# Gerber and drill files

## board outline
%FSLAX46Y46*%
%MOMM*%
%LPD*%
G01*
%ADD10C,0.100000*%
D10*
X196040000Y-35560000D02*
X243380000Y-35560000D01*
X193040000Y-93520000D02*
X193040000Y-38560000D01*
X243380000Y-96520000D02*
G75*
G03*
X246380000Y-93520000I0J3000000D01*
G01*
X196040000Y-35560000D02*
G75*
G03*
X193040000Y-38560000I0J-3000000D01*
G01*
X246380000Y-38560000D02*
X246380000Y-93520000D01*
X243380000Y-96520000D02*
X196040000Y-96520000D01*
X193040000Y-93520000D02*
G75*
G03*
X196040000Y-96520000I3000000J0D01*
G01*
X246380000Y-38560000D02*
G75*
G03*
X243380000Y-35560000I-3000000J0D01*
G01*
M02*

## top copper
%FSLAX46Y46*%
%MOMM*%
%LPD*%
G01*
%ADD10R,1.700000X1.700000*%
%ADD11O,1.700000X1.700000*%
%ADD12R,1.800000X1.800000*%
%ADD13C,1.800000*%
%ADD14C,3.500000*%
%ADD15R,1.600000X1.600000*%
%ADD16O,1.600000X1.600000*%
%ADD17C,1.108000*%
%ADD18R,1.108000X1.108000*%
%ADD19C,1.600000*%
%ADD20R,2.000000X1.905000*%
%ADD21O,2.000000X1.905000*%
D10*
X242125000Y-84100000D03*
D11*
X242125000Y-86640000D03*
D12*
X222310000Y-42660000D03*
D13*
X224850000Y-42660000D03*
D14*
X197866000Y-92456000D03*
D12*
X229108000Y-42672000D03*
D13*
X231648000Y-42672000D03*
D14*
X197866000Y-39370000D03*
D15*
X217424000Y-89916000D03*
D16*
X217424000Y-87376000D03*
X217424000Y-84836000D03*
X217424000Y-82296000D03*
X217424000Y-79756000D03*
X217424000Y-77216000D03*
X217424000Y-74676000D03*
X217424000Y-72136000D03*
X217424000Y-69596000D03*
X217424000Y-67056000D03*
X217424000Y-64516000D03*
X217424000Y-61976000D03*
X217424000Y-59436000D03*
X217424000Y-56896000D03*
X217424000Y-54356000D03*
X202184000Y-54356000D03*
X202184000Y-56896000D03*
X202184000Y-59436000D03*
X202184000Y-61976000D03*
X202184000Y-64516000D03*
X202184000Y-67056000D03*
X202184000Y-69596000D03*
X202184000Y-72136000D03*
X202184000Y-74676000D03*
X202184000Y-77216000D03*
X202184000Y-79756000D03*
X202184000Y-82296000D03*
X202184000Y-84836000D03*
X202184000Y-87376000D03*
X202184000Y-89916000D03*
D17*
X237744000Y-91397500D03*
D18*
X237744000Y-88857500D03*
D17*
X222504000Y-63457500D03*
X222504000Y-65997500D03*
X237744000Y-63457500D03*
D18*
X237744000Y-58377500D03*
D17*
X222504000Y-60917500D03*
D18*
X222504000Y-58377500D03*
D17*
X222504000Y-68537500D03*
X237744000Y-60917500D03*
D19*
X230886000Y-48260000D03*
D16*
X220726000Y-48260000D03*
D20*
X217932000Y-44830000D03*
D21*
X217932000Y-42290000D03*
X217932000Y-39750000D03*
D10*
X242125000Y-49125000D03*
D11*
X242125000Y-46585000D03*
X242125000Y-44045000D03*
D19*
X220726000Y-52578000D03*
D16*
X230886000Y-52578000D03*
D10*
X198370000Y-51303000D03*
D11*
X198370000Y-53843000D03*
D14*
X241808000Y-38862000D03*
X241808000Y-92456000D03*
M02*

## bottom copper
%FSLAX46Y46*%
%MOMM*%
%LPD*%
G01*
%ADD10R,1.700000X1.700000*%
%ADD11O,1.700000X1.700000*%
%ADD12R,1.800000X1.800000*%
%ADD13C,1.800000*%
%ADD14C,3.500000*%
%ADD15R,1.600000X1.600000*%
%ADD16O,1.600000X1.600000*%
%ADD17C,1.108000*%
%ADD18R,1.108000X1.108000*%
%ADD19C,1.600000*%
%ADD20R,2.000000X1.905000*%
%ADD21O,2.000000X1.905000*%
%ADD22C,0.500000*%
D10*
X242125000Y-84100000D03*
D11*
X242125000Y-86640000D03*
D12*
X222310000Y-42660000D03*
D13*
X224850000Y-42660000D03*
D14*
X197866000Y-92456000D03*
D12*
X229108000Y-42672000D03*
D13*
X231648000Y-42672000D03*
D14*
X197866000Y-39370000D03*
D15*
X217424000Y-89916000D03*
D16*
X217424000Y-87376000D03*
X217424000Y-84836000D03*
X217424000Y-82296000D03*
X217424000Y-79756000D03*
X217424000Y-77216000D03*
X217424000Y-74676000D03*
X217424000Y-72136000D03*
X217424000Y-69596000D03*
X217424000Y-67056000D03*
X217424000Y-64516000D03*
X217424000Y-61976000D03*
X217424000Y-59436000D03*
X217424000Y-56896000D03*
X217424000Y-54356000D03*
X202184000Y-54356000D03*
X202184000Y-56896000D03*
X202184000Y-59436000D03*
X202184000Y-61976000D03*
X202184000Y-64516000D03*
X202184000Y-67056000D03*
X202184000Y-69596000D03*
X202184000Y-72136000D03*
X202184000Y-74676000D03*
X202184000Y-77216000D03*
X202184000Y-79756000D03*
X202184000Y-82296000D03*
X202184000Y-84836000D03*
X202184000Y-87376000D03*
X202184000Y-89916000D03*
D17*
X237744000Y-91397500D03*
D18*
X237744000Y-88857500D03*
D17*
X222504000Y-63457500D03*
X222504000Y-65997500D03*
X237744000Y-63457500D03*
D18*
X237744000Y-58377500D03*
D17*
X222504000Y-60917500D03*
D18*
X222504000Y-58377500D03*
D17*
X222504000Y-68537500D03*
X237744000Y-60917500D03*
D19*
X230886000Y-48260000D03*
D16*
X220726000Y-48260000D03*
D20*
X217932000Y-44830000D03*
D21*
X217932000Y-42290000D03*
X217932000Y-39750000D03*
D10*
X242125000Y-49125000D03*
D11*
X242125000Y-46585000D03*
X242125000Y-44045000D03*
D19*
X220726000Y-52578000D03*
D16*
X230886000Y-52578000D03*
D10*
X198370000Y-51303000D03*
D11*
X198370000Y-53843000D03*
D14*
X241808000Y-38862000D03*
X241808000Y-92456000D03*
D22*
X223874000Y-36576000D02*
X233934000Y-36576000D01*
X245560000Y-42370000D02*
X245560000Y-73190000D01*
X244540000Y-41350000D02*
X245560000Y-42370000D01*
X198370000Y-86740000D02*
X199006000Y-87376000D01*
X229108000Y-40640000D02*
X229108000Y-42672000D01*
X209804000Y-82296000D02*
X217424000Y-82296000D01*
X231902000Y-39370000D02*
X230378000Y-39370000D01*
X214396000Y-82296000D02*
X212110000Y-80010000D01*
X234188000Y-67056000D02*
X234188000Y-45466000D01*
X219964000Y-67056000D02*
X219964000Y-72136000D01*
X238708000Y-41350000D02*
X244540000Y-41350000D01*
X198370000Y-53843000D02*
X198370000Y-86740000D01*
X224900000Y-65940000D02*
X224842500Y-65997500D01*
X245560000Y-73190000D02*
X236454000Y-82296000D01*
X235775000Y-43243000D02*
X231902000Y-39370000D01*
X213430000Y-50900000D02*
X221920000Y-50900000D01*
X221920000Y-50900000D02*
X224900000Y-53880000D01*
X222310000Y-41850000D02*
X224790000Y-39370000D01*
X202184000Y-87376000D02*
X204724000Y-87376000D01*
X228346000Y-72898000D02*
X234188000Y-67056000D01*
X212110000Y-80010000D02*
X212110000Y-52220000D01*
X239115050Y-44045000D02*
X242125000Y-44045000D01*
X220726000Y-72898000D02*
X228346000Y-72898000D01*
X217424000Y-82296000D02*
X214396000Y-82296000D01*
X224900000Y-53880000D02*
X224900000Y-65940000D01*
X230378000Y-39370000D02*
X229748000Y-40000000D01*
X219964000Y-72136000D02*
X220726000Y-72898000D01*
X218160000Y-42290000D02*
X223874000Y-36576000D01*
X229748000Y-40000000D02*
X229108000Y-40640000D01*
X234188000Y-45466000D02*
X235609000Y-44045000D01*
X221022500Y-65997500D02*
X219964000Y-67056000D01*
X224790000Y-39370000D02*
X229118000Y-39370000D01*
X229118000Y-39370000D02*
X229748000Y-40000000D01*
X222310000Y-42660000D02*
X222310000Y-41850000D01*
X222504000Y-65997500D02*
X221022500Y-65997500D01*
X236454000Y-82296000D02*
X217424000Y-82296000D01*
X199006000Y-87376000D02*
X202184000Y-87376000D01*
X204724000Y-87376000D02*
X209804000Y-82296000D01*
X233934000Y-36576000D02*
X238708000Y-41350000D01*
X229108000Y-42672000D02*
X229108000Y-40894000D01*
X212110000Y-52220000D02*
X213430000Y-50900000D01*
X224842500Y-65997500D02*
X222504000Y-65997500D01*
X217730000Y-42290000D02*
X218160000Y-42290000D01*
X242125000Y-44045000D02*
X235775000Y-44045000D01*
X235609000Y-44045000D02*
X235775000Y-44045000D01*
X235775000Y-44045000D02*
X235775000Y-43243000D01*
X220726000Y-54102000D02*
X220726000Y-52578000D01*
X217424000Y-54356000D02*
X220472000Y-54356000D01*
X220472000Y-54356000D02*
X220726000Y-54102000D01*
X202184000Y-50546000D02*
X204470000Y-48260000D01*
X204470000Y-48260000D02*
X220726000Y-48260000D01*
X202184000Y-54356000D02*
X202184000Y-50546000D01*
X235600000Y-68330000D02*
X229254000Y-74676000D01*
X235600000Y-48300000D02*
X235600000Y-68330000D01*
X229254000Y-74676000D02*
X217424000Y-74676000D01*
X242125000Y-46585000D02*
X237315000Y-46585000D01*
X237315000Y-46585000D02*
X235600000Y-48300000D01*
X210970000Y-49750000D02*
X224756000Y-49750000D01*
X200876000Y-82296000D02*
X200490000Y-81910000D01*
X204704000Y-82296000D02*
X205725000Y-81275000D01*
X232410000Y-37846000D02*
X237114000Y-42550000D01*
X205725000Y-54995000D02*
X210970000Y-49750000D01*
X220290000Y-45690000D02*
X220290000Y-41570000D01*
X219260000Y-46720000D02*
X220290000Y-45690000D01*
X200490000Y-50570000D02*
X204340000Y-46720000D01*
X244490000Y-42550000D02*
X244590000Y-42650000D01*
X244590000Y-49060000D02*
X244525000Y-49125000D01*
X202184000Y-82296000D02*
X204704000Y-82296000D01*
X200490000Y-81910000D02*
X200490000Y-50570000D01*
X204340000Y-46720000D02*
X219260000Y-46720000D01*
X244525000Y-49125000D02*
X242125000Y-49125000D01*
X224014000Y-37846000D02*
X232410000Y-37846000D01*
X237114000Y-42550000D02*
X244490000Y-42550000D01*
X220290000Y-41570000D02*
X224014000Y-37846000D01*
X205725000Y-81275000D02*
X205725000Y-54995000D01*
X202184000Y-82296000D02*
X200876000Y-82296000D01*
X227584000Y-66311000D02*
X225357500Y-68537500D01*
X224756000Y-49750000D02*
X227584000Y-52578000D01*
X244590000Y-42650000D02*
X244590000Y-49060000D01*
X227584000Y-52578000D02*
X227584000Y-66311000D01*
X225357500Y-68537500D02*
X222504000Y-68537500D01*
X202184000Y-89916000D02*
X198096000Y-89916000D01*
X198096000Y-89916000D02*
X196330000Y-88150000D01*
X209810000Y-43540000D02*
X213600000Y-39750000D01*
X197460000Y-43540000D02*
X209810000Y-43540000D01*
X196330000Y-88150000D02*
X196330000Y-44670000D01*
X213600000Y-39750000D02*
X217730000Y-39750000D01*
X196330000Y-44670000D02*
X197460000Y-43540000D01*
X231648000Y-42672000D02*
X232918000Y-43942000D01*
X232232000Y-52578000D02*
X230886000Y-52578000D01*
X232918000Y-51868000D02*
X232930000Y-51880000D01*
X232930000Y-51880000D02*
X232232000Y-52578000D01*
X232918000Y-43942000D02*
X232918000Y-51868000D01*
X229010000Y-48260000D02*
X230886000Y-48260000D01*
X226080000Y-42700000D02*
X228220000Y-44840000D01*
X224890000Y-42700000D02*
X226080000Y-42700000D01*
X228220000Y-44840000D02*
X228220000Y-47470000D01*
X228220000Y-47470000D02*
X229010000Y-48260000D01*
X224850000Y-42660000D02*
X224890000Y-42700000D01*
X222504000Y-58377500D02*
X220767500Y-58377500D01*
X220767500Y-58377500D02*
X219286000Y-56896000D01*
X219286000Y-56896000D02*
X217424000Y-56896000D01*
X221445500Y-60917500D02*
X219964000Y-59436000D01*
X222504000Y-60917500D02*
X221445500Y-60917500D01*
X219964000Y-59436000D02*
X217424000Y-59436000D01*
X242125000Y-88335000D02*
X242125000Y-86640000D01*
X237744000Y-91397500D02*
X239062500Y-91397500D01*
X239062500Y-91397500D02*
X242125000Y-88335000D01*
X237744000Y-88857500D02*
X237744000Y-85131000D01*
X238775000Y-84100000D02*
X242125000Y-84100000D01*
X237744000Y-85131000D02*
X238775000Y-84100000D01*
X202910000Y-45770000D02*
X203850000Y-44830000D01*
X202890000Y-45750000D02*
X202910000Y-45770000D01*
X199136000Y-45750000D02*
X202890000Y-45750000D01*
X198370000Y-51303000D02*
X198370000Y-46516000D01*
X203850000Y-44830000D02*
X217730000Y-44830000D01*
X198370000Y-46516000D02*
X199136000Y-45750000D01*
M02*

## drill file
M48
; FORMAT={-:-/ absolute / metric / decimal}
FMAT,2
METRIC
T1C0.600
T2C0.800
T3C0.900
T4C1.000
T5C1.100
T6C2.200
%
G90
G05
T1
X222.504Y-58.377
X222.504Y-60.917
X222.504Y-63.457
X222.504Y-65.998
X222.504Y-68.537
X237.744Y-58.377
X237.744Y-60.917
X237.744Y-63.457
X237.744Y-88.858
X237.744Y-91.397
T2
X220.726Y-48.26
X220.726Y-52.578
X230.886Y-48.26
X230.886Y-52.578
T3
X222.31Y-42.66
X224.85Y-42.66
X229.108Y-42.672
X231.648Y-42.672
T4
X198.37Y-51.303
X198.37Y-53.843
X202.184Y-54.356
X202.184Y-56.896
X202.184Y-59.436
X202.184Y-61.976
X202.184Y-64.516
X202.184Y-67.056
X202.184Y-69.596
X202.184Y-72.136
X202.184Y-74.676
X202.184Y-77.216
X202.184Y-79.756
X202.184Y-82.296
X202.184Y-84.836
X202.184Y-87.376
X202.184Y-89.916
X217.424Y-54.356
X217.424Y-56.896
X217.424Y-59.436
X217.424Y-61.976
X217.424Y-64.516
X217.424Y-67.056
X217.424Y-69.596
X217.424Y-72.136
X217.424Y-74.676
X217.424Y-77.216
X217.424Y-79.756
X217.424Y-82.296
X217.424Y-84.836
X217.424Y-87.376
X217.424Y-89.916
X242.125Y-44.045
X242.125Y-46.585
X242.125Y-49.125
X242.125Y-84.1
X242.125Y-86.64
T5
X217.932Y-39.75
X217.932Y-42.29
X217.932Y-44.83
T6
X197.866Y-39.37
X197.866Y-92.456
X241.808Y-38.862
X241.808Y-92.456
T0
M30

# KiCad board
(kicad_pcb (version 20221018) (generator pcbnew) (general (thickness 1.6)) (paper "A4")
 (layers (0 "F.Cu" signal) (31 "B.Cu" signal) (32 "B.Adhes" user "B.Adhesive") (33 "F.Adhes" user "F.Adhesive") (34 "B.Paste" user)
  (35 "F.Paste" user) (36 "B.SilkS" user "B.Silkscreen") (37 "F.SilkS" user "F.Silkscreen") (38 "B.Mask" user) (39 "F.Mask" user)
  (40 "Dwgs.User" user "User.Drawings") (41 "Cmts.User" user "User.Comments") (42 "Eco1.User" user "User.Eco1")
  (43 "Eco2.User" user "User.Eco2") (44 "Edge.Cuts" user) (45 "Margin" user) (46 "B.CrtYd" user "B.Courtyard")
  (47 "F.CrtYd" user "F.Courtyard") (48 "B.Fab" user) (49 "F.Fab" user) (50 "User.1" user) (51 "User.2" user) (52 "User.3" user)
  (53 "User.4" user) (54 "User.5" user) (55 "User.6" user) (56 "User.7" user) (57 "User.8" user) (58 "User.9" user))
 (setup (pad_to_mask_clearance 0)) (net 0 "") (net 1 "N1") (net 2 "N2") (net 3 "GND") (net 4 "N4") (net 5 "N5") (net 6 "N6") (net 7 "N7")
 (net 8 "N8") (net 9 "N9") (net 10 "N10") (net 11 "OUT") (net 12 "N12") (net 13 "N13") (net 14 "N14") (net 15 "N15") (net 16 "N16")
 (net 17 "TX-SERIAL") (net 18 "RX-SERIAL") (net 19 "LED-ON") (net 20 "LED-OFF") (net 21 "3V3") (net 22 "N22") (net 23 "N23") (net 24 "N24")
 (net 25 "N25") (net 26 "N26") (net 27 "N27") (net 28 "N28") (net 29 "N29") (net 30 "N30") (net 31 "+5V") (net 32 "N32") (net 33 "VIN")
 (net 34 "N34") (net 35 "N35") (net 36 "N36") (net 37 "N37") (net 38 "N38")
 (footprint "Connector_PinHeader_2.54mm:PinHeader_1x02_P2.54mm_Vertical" (layer "F.Cu") (at 242.125 84.1)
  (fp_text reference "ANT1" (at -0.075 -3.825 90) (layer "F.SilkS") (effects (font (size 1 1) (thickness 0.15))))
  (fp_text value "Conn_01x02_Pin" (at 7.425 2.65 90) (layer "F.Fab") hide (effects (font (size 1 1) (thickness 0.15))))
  (pad "1" thru_hole rect (at 0 0) (size 1.7 1.7) (drill 1) (layers "*.Cu" "*.Mask") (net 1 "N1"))
  (pad "2" thru_hole oval (at 0 2.54) (size 1.7 1.7) (drill 1) (layers "*.Cu" "*.Mask") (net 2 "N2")))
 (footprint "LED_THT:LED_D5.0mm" (layer "F.Cu") (at 222.31 42.66)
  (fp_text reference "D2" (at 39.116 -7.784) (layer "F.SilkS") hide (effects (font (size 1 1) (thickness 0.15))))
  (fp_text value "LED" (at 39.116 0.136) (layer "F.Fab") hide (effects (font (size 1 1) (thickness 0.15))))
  (pad "1" thru_hole rect (at 0 0) (size 1.8 1.8) (drill 0.9) (layers "*.Cu" "*.Mask") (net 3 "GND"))
  (pad "2" thru_hole circle (at 2.54 0) (size 1.8 1.8) (drill 0.9) (layers "*.Cu" "*.Mask") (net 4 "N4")))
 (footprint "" (layer "F.Cu") (at 197.866 92.456)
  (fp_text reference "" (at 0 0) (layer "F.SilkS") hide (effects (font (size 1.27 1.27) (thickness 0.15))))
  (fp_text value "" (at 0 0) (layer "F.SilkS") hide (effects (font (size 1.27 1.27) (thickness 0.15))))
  (pad "1" thru_hole circle (at 0 0) (size 3.5 3.5) (drill 2.2) (layers "*.Cu" "*.Mask")))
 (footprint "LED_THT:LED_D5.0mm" (layer "F.Cu") (at 229.108 42.672)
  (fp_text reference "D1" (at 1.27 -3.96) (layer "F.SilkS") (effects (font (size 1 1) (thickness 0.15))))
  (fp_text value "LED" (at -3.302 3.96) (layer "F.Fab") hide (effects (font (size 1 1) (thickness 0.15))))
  (pad "1" thru_hole rect (at 0 0) (size 1.8 1.8) (drill 0.9) (layers "*.Cu" "*.Mask") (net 3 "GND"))
  (pad "2" thru_hole circle (at 2.54 0) (size 1.8 1.8) (drill 0.9) (layers "*.Cu" "*.Mask") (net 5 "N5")))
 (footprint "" (layer "F.Cu") (at 197.866 39.37)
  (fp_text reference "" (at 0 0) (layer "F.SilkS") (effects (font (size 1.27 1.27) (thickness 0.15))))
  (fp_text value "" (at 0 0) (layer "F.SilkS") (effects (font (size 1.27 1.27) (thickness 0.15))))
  (pad "1" thru_hole circle (at 0 0) (size 3.5 3.5) (drill 2.2) (layers "*.Cu" "*.Mask")))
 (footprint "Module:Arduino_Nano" (layer "F.Cu") (at 217.424 89.916 180)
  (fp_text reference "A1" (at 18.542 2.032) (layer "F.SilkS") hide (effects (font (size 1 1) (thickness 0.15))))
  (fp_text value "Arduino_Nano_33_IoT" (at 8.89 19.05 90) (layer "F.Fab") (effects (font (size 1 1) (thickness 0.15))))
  (pad "1" thru_hole rect (at 0 0 180) (size 1.6 1.6) (drill 1) (layers "*.Cu" "*.Mask") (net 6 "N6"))
  (pad "2" thru_hole oval (at 0 2.54 180) (size 1.6 1.6) (drill 1) (layers "*.Cu" "*.Mask") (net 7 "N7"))
  (pad "3" thru_hole oval (at 0 5.08 180) (size 1.6 1.6) (drill 1) (layers "*.Cu" "*.Mask") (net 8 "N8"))
  (pad "4" thru_hole oval (at 0 7.62 180) (size 1.6 1.6) (drill 1) (layers "*.Cu" "*.Mask") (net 3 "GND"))
  (pad "5" thru_hole oval (at 0 10.16 180) (size 1.6 1.6) (drill 1) (layers "*.Cu" "*.Mask") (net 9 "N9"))
  (pad "6" thru_hole oval (at 0 12.7 180) (size 1.6 1.6) (drill 1) (layers "*.Cu" "*.Mask") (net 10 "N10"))
  (pad "7" thru_hole oval (at 0 15.24 180) (size 1.6 1.6) (drill 1) (layers "*.Cu" "*.Mask") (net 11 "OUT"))
  (pad "8" thru_hole oval (at 0 17.78 180) (size 1.6 1.6) (drill 1) (layers "*.Cu" "*.Mask") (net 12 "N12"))
  (pad "9" thru_hole oval (at 0 20.32 180) (size 1.6 1.6) (drill 1) (layers "*.Cu" "*.Mask") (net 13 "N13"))
  (pad "10" thru_hole oval (at 0 22.86 180) (size 1.6 1.6) (drill 1) (layers "*.Cu" "*.Mask") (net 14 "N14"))
  (pad "11" thru_hole oval (at 0 25.4 180) (size 1.6 1.6) (drill 1) (layers "*.Cu" "*.Mask") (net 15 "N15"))
  (pad "12" thru_hole oval (at 0 27.94 180) (size 1.6 1.6) (drill 1) (layers "*.Cu" "*.Mask") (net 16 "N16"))
  (pad "13" thru_hole oval (at 0 30.48 180) (size 1.6 1.6) (drill 1) (layers "*.Cu" "*.Mask") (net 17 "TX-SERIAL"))
  (pad "14" thru_hole oval (at 0 33.02 180) (size 1.6 1.6) (drill 1) (layers "*.Cu" "*.Mask") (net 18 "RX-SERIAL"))
  (pad "15" thru_hole oval (at 0 35.56 180) (size 1.6 1.6) (drill 1) (layers "*.Cu" "*.Mask") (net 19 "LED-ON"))
  (pad "16" thru_hole oval (at 15.24 35.56 180) (size 1.6 1.6) (drill 1) (layers "*.Cu" "*.Mask") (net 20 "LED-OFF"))
  (pad "17" thru_hole oval (at 15.24 33.02 180) (size 1.6 1.6) (drill 1) (layers "*.Cu" "*.Mask") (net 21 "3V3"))
  (pad "18" thru_hole oval (at 15.24 30.48 180) (size 1.6 1.6) (drill 1) (layers "*.Cu" "*.Mask") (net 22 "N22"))
  (pad "19" thru_hole oval (at 15.24 27.94 180) (size 1.6 1.6) (drill 1) (layers "*.Cu" "*.Mask") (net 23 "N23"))
  (pad "20" thru_hole oval (at 15.24 25.4 180) (size 1.6 1.6) (drill 1) (layers "*.Cu" "*.Mask") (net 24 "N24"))
  (pad "21" thru_hole oval (at 15.24 22.86 180) (size 1.6 1.6) (drill 1) (layers "*.Cu" "*.Mask") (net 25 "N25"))
  (pad "22" thru_hole oval (at 15.24 20.32 180) (size 1.6 1.6) (drill 1) (layers "*.Cu" "*.Mask") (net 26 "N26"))
  (pad "23" thru_hole oval (at 15.24 17.78 180) (size 1.6 1.6) (drill 1) (layers "*.Cu" "*.Mask") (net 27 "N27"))
  (pad "24" thru_hole oval (at 15.24 15.24 180) (size 1.6 1.6) (drill 1) (layers "*.Cu" "*.Mask") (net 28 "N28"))
  (pad "25" thru_hole oval (at 15.24 12.7 180) (size 1.6 1.6) (drill 1) (layers "*.Cu" "*.Mask") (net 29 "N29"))
  (pad "26" thru_hole oval (at 15.24 10.16 180) (size 1.6 1.6) (drill 1) (layers "*.Cu" "*.Mask") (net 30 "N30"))
  (pad "27" thru_hole oval (at 15.24 7.62 180) (size 1.6 1.6) (drill 1) (layers "*.Cu" "*.Mask") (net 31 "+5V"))
  (pad "28" thru_hole oval (at 15.24 5.08 180) (size 1.6 1.6) (drill 1) (layers "*.Cu" "*.Mask") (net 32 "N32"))
  (pad "29" thru_hole oval (at 15.24 2.54 180) (size 1.6 1.6) (drill 1) (layers "*.Cu" "*.Mask") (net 3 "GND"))
  (pad "30" thru_hole oval (at 15.24 0 180) (size 1.6 1.6) (drill 1) (layers "*.Cu" "*.Mask") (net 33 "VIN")))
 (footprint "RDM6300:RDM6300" (layer "F.Cu") (at 230.124 74.8875 90)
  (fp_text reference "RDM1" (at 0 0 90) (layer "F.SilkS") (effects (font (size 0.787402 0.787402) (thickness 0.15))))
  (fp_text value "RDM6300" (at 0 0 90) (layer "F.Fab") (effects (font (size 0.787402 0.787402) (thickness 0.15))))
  (pad "ANT1" thru_hole circle (at -16.51 7.62 90) (size 1.108 1.108) (drill 0.6) (layers "*.Cu" "*.Mask") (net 2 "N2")
   (solder_mask_margin 0.102))
  (pad "ANT2" thru_hole rect (at -13.97 7.62 90) (size 1.108 1.108) (drill 0.6) (layers "*.Cu" "*.Mask") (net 1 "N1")
   (solder_mask_margin 0.102))
  (pad "D0" thru_hole circle (at 11.43 -7.62 90) (size 1.108 1.108) (drill 0.6) (layers "*.Cu" "*.Mask") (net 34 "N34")
   (solder_mask_margin 0.102))
  (pad "GND" thru_hole circle (at 8.89 -7.62 90) (size 1.108 1.108) (drill 0.6) (layers "*.Cu" "*.Mask") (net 3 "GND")
   (solder_mask_margin 0.102))
  (pad "GND1" thru_hole circle (at 11.43 7.62 90) (size 1.108 1.108) (drill 0.6) (layers "*.Cu" "*.Mask") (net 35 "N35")
   (solder_mask_margin 0.102))
  (pad "LED" thru_hole rect (at 16.51 7.62 90) (size 1.108 1.108) (drill 0.6) (layers "*.Cu" "*.Mask") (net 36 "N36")
   (solder_mask_margin 0.102))
  (pad "RX" thru_hole circle (at 13.97 -7.62 90) (size 1.108 1.108) (drill 0.6) (layers "*.Cu" "*.Mask") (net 17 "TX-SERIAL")
   (solder_mask_margin 0.102))
  (pad "TX" thru_hole rect (at 16.51 -7.62 90) (size 1.108 1.108) (drill 0.6) (layers "*.Cu" "*.Mask") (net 18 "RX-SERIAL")
   (solder_mask_margin 0.102))
  (pad "VCC" thru_hole circle (at 6.35 -7.62 90) (size 1.108 1.108) (drill 0.6) (layers "*.Cu" "*.Mask") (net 31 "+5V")
   (solder_mask_margin 0.102))
  (pad "VCC1" thru_hole circle (at 13.97 7.62 90) (size 1.108 1.108) (drill 0.6) (layers "*.Cu" "*.Mask") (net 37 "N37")
   (solder_mask_margin 0.102)))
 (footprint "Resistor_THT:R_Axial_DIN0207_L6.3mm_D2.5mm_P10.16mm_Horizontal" (layer "F.Cu") (at 230.886 48.26 180)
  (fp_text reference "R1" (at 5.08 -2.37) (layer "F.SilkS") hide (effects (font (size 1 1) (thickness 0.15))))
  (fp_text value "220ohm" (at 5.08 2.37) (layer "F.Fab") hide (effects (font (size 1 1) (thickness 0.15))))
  (pad "1" thru_hole circle (at 0 0 180) (size 1.6 1.6) (drill 0.8) (layers "*.Cu" "*.Mask") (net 4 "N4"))
  (pad "2" thru_hole oval (at 10.16 0 180) (size 1.6 1.6) (drill 0.8) (layers "*.Cu" "*.Mask") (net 20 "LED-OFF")))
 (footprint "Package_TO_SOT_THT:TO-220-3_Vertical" (layer "F.Cu") (at 217.932 44.83 90)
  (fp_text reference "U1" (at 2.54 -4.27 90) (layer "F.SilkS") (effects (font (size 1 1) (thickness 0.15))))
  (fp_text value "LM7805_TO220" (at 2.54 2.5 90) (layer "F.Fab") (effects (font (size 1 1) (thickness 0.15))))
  (pad "1" thru_hole rect (at 0 0 90) (size 1.905 2) (drill 1.1) (layers "*.Cu" "*.Mask") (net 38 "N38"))
  (pad "2" thru_hole oval (at 2.54 0 90) (size 1.905 2) (drill 1.1) (layers "*.Cu" "*.Mask") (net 3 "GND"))
  (pad "3" thru_hole oval (at 5.08 0 90) (size 1.905 2) (drill 1.1) (layers "*.Cu" "*.Mask") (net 33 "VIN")))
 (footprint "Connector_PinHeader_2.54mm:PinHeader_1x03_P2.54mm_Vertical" (layer "F.Cu") (at 242.125 49.125 180)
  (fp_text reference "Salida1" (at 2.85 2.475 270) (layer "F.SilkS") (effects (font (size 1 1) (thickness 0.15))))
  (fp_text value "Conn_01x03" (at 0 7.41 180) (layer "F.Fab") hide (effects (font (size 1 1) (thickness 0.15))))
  (pad "1" thru_hole rect (at 0 0 180) (size 1.7 1.7) (drill 1) (layers "*.Cu" "*.Mask") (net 31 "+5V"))
  (pad "2" thru_hole oval (at 0 2.54 180) (size 1.7 1.7) (drill 1) (layers "*.Cu" "*.Mask") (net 11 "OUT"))
  (pad "3" thru_hole oval (at 0 5.08 180) (size 1.7 1.7) (drill 1) (layers "*.Cu" "*.Mask") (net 3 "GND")))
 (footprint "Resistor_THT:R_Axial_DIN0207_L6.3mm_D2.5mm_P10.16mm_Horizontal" (layer "F.Cu") (at 220.726 52.578)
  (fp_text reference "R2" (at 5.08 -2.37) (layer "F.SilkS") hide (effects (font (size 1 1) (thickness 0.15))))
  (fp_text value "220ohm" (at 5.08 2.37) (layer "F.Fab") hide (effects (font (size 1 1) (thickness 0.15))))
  (pad "1" thru_hole circle (at 0 0) (size 1.6 1.6) (drill 0.8) (layers "*.Cu" "*.Mask") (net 19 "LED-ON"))
  (pad "2" thru_hole oval (at 10.16 0) (size 1.6 1.6) (drill 0.8) (layers "*.Cu" "*.Mask") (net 5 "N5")))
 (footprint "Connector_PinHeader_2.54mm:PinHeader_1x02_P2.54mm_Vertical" (layer "F.Cu") (at 198.37 51.303)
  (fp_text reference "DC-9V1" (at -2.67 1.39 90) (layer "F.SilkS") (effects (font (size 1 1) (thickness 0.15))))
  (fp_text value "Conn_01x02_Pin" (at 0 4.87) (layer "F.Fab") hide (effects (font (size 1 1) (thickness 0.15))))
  (pad "1" thru_hole rect (at 0 0) (size 1.7 1.7) (drill 1) (layers "*.Cu" "*.Mask") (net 38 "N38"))
  (pad "2" thru_hole oval (at 0 2.54) (size 1.7 1.7) (drill 1) (layers "*.Cu" "*.Mask") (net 3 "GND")))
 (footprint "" (layer "F.Cu") (at 241.808 38.862)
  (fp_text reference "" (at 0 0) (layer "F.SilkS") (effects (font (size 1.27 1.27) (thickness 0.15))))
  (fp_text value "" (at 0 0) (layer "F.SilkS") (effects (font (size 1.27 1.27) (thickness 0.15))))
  (pad "1" thru_hole circle (at 0 0) (size 3.5 3.5) (drill 2.2) (layers "*.Cu" "*.Mask")))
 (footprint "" (layer "F.Cu") (at 241.808 92.456)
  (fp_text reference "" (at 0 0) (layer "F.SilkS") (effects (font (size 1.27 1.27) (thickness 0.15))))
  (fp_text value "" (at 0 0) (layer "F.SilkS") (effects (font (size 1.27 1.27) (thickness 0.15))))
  (pad "1" thru_hole circle (at 0 0) (size 3.5 3.5) (drill 2.2) (layers "*.Cu" "*.Mask")))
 (gr_line (start 196.04 35.56) (end 243.38 35.56) (stroke (width 0.1) (type default)) (layer "Edge.Cuts"))
 (gr_line (start 193.04 93.52) (end 193.04 38.56) (stroke (width 0.1) (type default)) (layer "Edge.Cuts"))
 (gr_arc (start 246.38 93.52) (mid 245.50132 95.64132) (end 243.38 96.52) (stroke (width 0.1) (type default)) (layer "Edge.Cuts"))
 (gr_arc (start 193.04 38.56) (mid 193.91868 36.43868) (end 196.04 35.56) (stroke (width 0.1) (type default)) (layer "Edge.Cuts"))
 (gr_line (start 246.38 38.56) (end 246.38 93.52) (stroke (width 0.1) (type default)) (layer "Edge.Cuts"))
 (gr_line (start 243.38 96.52) (end 196.04 96.52) (stroke (width 0.1) (type default)) (layer "Edge.Cuts"))
 (gr_arc (start 196.04 96.52) (mid 193.91868 95.64132) (end 193.04 93.52) (stroke (width 0.1) (type default)) (layer "Edge.Cuts"))
 (gr_arc (start 243.38 35.56) (mid 245.50132 36.43868) (end 246.38 38.56) (stroke (width 0.1) (type default)) (layer "Edge.Cuts"))
 (segment (start 223.874 36.576) (end 233.934 36.576) (width 0.5) (layer "B.Cu") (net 3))
 (segment (start 245.56 42.37) (end 245.56 73.19) (width 0.5) (layer "B.Cu") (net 3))
 (segment (start 244.54 41.35) (end 245.56 42.37) (width 0.5) (layer "B.Cu") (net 3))
 (segment (start 198.37 86.74) (end 199.006 87.376) (width 0.5) (layer "B.Cu") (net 3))
 (segment (start 229.108 40.64) (end 229.108 42.672) (width 0.5) (layer "B.Cu") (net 3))
 (segment (start 209.804 82.296) (end 217.424 82.296) (width 0.5) (layer "B.Cu") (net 3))
 (segment (start 231.902 39.37) (end 230.378 39.37) (width 0.5) (layer "B.Cu") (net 3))
 (segment (start 214.396 82.296) (end 212.11 80.01) (width 0.5) (layer "B.Cu") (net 3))
 (segment (start 234.188 67.056) (end 234.188 45.466) (width 0.5) (layer "B.Cu") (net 3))
 (segment (start 219.964 67.056) (end 219.964 72.136) (width 0.5) (layer "B.Cu") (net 3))
 (segment (start 238.708 41.35) (end 244.54 41.35) (width 0.5) (layer "B.Cu") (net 3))
 (segment (start 198.37 53.843) (end 198.37 86.74) (width 0.5) (layer "B.Cu") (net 3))
 (segment (start 224.9 65.94) (end 224.8425 65.9975) (width 0.5) (layer "B.Cu") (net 3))
 (segment (start 245.56 73.19) (end 236.454 82.296) (width 0.5) (layer "B.Cu") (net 3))
 (segment (start 235.775 43.243) (end 231.902 39.37) (width 0.5) (layer "B.Cu") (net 3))
 (segment (start 213.43 50.9) (end 221.92 50.9) (width 0.5) (layer "B.Cu") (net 3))
 (segment (start 221.92 50.9) (end 224.9 53.88) (width 0.5) (layer "B.Cu") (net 3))
 (segment (start 222.31 41.85) (end 224.79 39.37) (width 0.5) (layer "B.Cu") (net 3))
 (segment (start 202.184 87.376) (end 204.724 87.376) (width 0.5) (layer "B.Cu") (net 3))
 (segment (start 228.346 72.898) (end 234.188 67.056) (width 0.5) (layer "B.Cu") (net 3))
 (segment (start 212.11 80.01) (end 212.11 52.22) (width 0.5) (layer "B.Cu") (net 3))
 (segment (start 239.11505 44.045) (end 242.125 44.045) (width 0.5) (layer "B.Cu") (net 3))
 (segment (start 220.726 72.898) (end 228.346 72.898) (width 0.5) (layer "B.Cu") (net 3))
 (segment (start 217.424 82.296) (end 214.396 82.296) (width 0.5) (layer "B.Cu") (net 3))
 (segment (start 224.9 53.88) (end 224.9 65.94) (width 0.5) (layer "B.Cu") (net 3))
 (segment (start 230.378 39.37) (end 229.748 40) (width 0.5) (layer "B.Cu") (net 3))
 (segment (start 219.964 72.136) (end 220.726 72.898) (width 0.5) (layer "B.Cu") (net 3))
 (segment (start 218.16 42.29) (end 223.874 36.576) (width 0.5) (layer "B.Cu") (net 3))
 (segment (start 229.748 40) (end 229.108 40.64) (width 0.5) (layer "B.Cu") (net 3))
 (segment (start 234.188 45.466) (end 235.609 44.045) (width 0.5) (layer "B.Cu") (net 3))
 (segment (start 221.0225 65.9975) (end 219.964 67.056) (width 0.5) (layer "B.Cu") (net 3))
 (segment (start 224.79 39.37) (end 229.118 39.37) (width 0.5) (layer "B.Cu") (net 3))
 (segment (start 229.118 39.37) (end 229.748 40) (width 0.5) (layer "B.Cu") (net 3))
 (segment (start 222.31 42.66) (end 222.31 41.85) (width 0.5) (layer "B.Cu") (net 3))
 (segment (start 222.504 65.9975) (end 221.0225 65.9975) (width 0.5) (layer "B.Cu") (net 3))
 (segment (start 236.454 82.296) (end 217.424 82.296) (width 0.5) (layer "B.Cu") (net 3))
 (segment (start 199.006 87.376) (end 202.184 87.376) (width 0.5) (layer "B.Cu") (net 3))
 (segment (start 204.724 87.376) (end 209.804 82.296) (width 0.5) (layer "B.Cu") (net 3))
 (segment (start 233.934 36.576) (end 238.708 41.35) (width 0.5) (layer "B.Cu") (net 3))
 (segment (start 229.108 42.672) (end 229.108 40.894) (width 0.5) (layer "B.Cu") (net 3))
 (segment (start 212.11 52.22) (end 213.43 50.9) (width 0.5) (layer "B.Cu") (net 3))
 (segment (start 224.8425 65.9975) (end 222.504 65.9975) (width 0.5) (layer "B.Cu") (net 3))
 (segment (start 217.73 42.29) (end 218.16 42.29) (width 0.5) (layer "B.Cu") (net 3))
 (segment (start 242.125 44.045) (end 235.775 44.045) (width 0.5) (layer "B.Cu") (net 3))
 (segment (start 235.609 44.045) (end 235.775 44.045) (width 0.5) (layer "B.Cu") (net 3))
 (segment (start 235.775 44.045) (end 235.775 43.243) (width 0.5) (layer "B.Cu") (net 3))
 (segment (start 220.726 54.102) (end 220.726 52.578) (width 0.5) (layer "B.Cu") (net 19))
 (segment (start 217.424 54.356) (end 220.472 54.356) (width 0.5) (layer "B.Cu") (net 19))
 (segment (start 220.472 54.356) (end 220.726 54.102) (width 0.5) (layer "B.Cu") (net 19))
 (segment (start 202.184 50.546) (end 204.47 48.26) (width 0.5) (layer "B.Cu") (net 20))
 (segment (start 204.47 48.26) (end 220.726 48.26) (width 0.5) (layer "B.Cu") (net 20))
 (segment (start 202.184 54.356) (end 202.184 50.546) (width 0.5) (layer "B.Cu") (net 20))
 (segment (start 235.6 68.33) (end 229.254 74.676) (width 0.5) (layer "B.Cu") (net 11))
 (segment (start 235.6 48.3) (end 235.6 68.33) (width 0.5) (layer "B.Cu") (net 11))
 (segment (start 229.254 74.676) (end 217.424 74.676) (width 0.5) (layer "B.Cu") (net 11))
 (segment (start 242.125 46.585) (end 237.315 46.585) (width 0.5) (layer "B.Cu") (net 11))
 (segment (start 237.315 46.585) (end 235.6 48.3) (width 0.5) (layer "B.Cu") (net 11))
 (segment (start 210.97 49.75) (end 224.756 49.75) (width 0.5) (layer "B.Cu") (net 31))
 (segment (start 200.876 82.296) (end 200.49 81.91) (width 0.5) (layer "B.Cu") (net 31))
 (segment (start 204.704 82.296) (end 205.725 81.275) (width 0.5) (layer "B.Cu") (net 31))
 (segment (start 232.41 37.846) (end 237.114 42.55) (width 0.5) (layer "B.Cu") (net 31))
 (segment (start 205.725 54.995) (end 210.97 49.75) (width 0.5) (layer "B.Cu") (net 31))
 (segment (start 220.29 45.69) (end 220.29 41.57) (width 0.5) (layer "B.Cu") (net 31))
 (segment (start 219.26 46.72) (end 220.29 45.69) (width 0.5) (layer "B.Cu") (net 31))
 (segment (start 200.49 50.57) (end 204.34 46.72) (width 0.5) (layer "B.Cu") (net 31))
 (segment (start 244.49 42.55) (end 244.59 42.65) (width 0.5) (layer "B.Cu") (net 31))
 (segment (start 244.59 49.06) (end 244.525 49.125) (width 0.5) (layer "B.Cu") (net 31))
 (segment (start 202.184 82.296) (end 204.704 82.296) (width 0.5) (layer "B.Cu") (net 31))
 (segment (start 200.49 81.91) (end 200.49 50.57) (width 0.5) (layer "B.Cu") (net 31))
 (segment (start 204.34 46.72) (end 219.26 46.72) (width 0.5) (layer "B.Cu") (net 31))
 (segment (start 244.525 49.125) (end 242.125 49.125) (width 0.5) (layer "B.Cu") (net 31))
 (segment (start 224.014 37.846) (end 232.41 37.846) (width 0.5) (layer "B.Cu") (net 31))
 (segment (start 237.114 42.55) (end 244.49 42.55) (width 0.5) (layer "B.Cu") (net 31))
 (segment (start 220.29 41.57) (end 224.014 37.846) (width 0.5) (layer "B.Cu") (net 31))
 (segment (start 205.725 81.275) (end 205.725 54.995) (width 0.5) (layer "B.Cu") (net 31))
 (segment (start 202.184 82.296) (end 200.876 82.296) (width 0.5) (layer "B.Cu") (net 31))
 (segment (start 227.584 66.311) (end 225.3575 68.5375) (width 0.5) (layer "B.Cu") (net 31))
 (segment (start 224.756 49.75) (end 227.584 52.578) (width 0.5) (layer "B.Cu") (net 31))
 (segment (start 244.59 42.65) (end 244.59 49.06) (width 0.5) (layer "B.Cu") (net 31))
 (segment (start 227.584 52.578) (end 227.584 66.311) (width 0.5) (layer "B.Cu") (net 31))
 (segment (start 225.3575 68.5375) (end 222.504 68.5375) (width 0.5) (layer "B.Cu") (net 31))
 (segment (start 202.184 89.916) (end 198.096 89.916) (width 0.5) (layer "B.Cu") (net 33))
 (segment (start 198.096 89.916) (end 196.33 88.15) (width 0.5) (layer "B.Cu") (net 33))
 (segment (start 209.81 43.54) (end 213.6 39.75) (width 0.5) (layer "B.Cu") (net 33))
 (segment (start 197.46 43.54) (end 209.81 43.54) (width 0.5) (layer "B.Cu") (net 33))
 (segment (start 196.33 88.15) (end 196.33 44.67) (width 0.5) (layer "B.Cu") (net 33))
 (segment (start 213.6 39.75) (end 217.73 39.75) (width 0.5) (layer "B.Cu") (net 33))
 (segment (start 196.33 44.67) (end 197.46 43.54) (width 0.5) (layer "B.Cu") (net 33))
 (segment (start 231.648 42.672) (end 232.918 43.942) (width 0.5) (layer "B.Cu") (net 5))
 (segment (start 232.232 52.578) (end 230.886 52.578) (width 0.5) (layer "B.Cu") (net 5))
 (segment (start 232.918 51.868) (end 232.93 51.88) (width 0.5) (layer "B.Cu") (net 5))
 (segment (start 232.93 51.88) (end 232.232 52.578) (width 0.5) (layer "B.Cu") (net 5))
 (segment (start 232.918 43.942) (end 232.918 51.868) (width 0.5) (layer "B.Cu") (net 5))
 (segment (start 229.01 48.26) (end 230.886 48.26) (width 0.5) (layer "B.Cu") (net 4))
 (segment (start 226.08 42.7) (end 228.22 44.84) (width 0.5) (layer "B.Cu") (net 4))
 (segment (start 224.89 42.7) (end 226.08 42.7) (width 0.5) (layer "B.Cu") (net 4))
 (segment (start 228.22 44.84) (end 228.22 47.47) (width 0.5) (layer "B.Cu") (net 4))
 (segment (start 228.22 47.47) (end 229.01 48.26) (width 0.5) (layer "B.Cu") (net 4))
 (segment (start 224.85 42.66) (end 224.89 42.7) (width 0.5) (layer "B.Cu") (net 4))
 (segment (start 222.504 58.3775) (end 220.7675 58.3775) (width 0.5) (layer "B.Cu") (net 18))
 (segment (start 220.7675 58.3775) (end 219.286 56.896) (width 0.5) (layer "B.Cu") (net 18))
 (segment (start 219.286 56.896) (end 217.424 56.896) (width 0.5) (layer "B.Cu") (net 18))
 (segment (start 221.4455 60.9175) (end 219.964 59.436) (width 0.5) (layer "B.Cu") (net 17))
 (segment (start 222.504 60.9175) (end 221.4455 60.9175) (width 0.5) (layer "B.Cu") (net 17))
 (segment (start 219.964 59.436) (end 217.424 59.436) (width 0.5) (layer "B.Cu") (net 17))
 (segment (start 242.125 88.335) (end 242.125 86.64) (width 0.5) (layer "B.Cu") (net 2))
 (segment (start 237.744 91.3975) (end 239.0625 91.3975) (width 0.5) (layer "B.Cu") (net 2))
 (segment (start 239.0625 91.3975) (end 242.125 88.335) (width 0.5) (layer "B.Cu") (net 2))
 (segment (start 237.744 88.8575) (end 237.744 85.131) (width 0.5) (layer "B.Cu") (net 1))
 (segment (start 238.775 84.1) (end 242.125 84.1) (width 0.5) (layer "B.Cu") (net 1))
 (segment (start 237.744 85.131) (end 238.775 84.1) (width 0.5) (layer "B.Cu") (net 1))
 (segment (start 202.91 45.77) (end 203.85 44.83) (width 0.5) (layer "B.Cu") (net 38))
 (segment (start 202.89 45.75) (end 202.91 45.77) (width 0.5) (layer "B.Cu") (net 38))
 (segment (start 199.136 45.75) (end 202.89 45.75) (width 0.5) (layer "B.Cu") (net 38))
 (segment (start 198.37 51.303) (end 198.37 46.516) (width 0.5) (layer "B.Cu") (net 38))
 (segment (start 203.85 44.83) (end 217.73 44.83) (width 0.5) (layer "B.Cu") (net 38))
 (segment (start 198.37 46.516) (end 199.136 45.75) (width 0.5) (layer "B.Cu") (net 38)))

